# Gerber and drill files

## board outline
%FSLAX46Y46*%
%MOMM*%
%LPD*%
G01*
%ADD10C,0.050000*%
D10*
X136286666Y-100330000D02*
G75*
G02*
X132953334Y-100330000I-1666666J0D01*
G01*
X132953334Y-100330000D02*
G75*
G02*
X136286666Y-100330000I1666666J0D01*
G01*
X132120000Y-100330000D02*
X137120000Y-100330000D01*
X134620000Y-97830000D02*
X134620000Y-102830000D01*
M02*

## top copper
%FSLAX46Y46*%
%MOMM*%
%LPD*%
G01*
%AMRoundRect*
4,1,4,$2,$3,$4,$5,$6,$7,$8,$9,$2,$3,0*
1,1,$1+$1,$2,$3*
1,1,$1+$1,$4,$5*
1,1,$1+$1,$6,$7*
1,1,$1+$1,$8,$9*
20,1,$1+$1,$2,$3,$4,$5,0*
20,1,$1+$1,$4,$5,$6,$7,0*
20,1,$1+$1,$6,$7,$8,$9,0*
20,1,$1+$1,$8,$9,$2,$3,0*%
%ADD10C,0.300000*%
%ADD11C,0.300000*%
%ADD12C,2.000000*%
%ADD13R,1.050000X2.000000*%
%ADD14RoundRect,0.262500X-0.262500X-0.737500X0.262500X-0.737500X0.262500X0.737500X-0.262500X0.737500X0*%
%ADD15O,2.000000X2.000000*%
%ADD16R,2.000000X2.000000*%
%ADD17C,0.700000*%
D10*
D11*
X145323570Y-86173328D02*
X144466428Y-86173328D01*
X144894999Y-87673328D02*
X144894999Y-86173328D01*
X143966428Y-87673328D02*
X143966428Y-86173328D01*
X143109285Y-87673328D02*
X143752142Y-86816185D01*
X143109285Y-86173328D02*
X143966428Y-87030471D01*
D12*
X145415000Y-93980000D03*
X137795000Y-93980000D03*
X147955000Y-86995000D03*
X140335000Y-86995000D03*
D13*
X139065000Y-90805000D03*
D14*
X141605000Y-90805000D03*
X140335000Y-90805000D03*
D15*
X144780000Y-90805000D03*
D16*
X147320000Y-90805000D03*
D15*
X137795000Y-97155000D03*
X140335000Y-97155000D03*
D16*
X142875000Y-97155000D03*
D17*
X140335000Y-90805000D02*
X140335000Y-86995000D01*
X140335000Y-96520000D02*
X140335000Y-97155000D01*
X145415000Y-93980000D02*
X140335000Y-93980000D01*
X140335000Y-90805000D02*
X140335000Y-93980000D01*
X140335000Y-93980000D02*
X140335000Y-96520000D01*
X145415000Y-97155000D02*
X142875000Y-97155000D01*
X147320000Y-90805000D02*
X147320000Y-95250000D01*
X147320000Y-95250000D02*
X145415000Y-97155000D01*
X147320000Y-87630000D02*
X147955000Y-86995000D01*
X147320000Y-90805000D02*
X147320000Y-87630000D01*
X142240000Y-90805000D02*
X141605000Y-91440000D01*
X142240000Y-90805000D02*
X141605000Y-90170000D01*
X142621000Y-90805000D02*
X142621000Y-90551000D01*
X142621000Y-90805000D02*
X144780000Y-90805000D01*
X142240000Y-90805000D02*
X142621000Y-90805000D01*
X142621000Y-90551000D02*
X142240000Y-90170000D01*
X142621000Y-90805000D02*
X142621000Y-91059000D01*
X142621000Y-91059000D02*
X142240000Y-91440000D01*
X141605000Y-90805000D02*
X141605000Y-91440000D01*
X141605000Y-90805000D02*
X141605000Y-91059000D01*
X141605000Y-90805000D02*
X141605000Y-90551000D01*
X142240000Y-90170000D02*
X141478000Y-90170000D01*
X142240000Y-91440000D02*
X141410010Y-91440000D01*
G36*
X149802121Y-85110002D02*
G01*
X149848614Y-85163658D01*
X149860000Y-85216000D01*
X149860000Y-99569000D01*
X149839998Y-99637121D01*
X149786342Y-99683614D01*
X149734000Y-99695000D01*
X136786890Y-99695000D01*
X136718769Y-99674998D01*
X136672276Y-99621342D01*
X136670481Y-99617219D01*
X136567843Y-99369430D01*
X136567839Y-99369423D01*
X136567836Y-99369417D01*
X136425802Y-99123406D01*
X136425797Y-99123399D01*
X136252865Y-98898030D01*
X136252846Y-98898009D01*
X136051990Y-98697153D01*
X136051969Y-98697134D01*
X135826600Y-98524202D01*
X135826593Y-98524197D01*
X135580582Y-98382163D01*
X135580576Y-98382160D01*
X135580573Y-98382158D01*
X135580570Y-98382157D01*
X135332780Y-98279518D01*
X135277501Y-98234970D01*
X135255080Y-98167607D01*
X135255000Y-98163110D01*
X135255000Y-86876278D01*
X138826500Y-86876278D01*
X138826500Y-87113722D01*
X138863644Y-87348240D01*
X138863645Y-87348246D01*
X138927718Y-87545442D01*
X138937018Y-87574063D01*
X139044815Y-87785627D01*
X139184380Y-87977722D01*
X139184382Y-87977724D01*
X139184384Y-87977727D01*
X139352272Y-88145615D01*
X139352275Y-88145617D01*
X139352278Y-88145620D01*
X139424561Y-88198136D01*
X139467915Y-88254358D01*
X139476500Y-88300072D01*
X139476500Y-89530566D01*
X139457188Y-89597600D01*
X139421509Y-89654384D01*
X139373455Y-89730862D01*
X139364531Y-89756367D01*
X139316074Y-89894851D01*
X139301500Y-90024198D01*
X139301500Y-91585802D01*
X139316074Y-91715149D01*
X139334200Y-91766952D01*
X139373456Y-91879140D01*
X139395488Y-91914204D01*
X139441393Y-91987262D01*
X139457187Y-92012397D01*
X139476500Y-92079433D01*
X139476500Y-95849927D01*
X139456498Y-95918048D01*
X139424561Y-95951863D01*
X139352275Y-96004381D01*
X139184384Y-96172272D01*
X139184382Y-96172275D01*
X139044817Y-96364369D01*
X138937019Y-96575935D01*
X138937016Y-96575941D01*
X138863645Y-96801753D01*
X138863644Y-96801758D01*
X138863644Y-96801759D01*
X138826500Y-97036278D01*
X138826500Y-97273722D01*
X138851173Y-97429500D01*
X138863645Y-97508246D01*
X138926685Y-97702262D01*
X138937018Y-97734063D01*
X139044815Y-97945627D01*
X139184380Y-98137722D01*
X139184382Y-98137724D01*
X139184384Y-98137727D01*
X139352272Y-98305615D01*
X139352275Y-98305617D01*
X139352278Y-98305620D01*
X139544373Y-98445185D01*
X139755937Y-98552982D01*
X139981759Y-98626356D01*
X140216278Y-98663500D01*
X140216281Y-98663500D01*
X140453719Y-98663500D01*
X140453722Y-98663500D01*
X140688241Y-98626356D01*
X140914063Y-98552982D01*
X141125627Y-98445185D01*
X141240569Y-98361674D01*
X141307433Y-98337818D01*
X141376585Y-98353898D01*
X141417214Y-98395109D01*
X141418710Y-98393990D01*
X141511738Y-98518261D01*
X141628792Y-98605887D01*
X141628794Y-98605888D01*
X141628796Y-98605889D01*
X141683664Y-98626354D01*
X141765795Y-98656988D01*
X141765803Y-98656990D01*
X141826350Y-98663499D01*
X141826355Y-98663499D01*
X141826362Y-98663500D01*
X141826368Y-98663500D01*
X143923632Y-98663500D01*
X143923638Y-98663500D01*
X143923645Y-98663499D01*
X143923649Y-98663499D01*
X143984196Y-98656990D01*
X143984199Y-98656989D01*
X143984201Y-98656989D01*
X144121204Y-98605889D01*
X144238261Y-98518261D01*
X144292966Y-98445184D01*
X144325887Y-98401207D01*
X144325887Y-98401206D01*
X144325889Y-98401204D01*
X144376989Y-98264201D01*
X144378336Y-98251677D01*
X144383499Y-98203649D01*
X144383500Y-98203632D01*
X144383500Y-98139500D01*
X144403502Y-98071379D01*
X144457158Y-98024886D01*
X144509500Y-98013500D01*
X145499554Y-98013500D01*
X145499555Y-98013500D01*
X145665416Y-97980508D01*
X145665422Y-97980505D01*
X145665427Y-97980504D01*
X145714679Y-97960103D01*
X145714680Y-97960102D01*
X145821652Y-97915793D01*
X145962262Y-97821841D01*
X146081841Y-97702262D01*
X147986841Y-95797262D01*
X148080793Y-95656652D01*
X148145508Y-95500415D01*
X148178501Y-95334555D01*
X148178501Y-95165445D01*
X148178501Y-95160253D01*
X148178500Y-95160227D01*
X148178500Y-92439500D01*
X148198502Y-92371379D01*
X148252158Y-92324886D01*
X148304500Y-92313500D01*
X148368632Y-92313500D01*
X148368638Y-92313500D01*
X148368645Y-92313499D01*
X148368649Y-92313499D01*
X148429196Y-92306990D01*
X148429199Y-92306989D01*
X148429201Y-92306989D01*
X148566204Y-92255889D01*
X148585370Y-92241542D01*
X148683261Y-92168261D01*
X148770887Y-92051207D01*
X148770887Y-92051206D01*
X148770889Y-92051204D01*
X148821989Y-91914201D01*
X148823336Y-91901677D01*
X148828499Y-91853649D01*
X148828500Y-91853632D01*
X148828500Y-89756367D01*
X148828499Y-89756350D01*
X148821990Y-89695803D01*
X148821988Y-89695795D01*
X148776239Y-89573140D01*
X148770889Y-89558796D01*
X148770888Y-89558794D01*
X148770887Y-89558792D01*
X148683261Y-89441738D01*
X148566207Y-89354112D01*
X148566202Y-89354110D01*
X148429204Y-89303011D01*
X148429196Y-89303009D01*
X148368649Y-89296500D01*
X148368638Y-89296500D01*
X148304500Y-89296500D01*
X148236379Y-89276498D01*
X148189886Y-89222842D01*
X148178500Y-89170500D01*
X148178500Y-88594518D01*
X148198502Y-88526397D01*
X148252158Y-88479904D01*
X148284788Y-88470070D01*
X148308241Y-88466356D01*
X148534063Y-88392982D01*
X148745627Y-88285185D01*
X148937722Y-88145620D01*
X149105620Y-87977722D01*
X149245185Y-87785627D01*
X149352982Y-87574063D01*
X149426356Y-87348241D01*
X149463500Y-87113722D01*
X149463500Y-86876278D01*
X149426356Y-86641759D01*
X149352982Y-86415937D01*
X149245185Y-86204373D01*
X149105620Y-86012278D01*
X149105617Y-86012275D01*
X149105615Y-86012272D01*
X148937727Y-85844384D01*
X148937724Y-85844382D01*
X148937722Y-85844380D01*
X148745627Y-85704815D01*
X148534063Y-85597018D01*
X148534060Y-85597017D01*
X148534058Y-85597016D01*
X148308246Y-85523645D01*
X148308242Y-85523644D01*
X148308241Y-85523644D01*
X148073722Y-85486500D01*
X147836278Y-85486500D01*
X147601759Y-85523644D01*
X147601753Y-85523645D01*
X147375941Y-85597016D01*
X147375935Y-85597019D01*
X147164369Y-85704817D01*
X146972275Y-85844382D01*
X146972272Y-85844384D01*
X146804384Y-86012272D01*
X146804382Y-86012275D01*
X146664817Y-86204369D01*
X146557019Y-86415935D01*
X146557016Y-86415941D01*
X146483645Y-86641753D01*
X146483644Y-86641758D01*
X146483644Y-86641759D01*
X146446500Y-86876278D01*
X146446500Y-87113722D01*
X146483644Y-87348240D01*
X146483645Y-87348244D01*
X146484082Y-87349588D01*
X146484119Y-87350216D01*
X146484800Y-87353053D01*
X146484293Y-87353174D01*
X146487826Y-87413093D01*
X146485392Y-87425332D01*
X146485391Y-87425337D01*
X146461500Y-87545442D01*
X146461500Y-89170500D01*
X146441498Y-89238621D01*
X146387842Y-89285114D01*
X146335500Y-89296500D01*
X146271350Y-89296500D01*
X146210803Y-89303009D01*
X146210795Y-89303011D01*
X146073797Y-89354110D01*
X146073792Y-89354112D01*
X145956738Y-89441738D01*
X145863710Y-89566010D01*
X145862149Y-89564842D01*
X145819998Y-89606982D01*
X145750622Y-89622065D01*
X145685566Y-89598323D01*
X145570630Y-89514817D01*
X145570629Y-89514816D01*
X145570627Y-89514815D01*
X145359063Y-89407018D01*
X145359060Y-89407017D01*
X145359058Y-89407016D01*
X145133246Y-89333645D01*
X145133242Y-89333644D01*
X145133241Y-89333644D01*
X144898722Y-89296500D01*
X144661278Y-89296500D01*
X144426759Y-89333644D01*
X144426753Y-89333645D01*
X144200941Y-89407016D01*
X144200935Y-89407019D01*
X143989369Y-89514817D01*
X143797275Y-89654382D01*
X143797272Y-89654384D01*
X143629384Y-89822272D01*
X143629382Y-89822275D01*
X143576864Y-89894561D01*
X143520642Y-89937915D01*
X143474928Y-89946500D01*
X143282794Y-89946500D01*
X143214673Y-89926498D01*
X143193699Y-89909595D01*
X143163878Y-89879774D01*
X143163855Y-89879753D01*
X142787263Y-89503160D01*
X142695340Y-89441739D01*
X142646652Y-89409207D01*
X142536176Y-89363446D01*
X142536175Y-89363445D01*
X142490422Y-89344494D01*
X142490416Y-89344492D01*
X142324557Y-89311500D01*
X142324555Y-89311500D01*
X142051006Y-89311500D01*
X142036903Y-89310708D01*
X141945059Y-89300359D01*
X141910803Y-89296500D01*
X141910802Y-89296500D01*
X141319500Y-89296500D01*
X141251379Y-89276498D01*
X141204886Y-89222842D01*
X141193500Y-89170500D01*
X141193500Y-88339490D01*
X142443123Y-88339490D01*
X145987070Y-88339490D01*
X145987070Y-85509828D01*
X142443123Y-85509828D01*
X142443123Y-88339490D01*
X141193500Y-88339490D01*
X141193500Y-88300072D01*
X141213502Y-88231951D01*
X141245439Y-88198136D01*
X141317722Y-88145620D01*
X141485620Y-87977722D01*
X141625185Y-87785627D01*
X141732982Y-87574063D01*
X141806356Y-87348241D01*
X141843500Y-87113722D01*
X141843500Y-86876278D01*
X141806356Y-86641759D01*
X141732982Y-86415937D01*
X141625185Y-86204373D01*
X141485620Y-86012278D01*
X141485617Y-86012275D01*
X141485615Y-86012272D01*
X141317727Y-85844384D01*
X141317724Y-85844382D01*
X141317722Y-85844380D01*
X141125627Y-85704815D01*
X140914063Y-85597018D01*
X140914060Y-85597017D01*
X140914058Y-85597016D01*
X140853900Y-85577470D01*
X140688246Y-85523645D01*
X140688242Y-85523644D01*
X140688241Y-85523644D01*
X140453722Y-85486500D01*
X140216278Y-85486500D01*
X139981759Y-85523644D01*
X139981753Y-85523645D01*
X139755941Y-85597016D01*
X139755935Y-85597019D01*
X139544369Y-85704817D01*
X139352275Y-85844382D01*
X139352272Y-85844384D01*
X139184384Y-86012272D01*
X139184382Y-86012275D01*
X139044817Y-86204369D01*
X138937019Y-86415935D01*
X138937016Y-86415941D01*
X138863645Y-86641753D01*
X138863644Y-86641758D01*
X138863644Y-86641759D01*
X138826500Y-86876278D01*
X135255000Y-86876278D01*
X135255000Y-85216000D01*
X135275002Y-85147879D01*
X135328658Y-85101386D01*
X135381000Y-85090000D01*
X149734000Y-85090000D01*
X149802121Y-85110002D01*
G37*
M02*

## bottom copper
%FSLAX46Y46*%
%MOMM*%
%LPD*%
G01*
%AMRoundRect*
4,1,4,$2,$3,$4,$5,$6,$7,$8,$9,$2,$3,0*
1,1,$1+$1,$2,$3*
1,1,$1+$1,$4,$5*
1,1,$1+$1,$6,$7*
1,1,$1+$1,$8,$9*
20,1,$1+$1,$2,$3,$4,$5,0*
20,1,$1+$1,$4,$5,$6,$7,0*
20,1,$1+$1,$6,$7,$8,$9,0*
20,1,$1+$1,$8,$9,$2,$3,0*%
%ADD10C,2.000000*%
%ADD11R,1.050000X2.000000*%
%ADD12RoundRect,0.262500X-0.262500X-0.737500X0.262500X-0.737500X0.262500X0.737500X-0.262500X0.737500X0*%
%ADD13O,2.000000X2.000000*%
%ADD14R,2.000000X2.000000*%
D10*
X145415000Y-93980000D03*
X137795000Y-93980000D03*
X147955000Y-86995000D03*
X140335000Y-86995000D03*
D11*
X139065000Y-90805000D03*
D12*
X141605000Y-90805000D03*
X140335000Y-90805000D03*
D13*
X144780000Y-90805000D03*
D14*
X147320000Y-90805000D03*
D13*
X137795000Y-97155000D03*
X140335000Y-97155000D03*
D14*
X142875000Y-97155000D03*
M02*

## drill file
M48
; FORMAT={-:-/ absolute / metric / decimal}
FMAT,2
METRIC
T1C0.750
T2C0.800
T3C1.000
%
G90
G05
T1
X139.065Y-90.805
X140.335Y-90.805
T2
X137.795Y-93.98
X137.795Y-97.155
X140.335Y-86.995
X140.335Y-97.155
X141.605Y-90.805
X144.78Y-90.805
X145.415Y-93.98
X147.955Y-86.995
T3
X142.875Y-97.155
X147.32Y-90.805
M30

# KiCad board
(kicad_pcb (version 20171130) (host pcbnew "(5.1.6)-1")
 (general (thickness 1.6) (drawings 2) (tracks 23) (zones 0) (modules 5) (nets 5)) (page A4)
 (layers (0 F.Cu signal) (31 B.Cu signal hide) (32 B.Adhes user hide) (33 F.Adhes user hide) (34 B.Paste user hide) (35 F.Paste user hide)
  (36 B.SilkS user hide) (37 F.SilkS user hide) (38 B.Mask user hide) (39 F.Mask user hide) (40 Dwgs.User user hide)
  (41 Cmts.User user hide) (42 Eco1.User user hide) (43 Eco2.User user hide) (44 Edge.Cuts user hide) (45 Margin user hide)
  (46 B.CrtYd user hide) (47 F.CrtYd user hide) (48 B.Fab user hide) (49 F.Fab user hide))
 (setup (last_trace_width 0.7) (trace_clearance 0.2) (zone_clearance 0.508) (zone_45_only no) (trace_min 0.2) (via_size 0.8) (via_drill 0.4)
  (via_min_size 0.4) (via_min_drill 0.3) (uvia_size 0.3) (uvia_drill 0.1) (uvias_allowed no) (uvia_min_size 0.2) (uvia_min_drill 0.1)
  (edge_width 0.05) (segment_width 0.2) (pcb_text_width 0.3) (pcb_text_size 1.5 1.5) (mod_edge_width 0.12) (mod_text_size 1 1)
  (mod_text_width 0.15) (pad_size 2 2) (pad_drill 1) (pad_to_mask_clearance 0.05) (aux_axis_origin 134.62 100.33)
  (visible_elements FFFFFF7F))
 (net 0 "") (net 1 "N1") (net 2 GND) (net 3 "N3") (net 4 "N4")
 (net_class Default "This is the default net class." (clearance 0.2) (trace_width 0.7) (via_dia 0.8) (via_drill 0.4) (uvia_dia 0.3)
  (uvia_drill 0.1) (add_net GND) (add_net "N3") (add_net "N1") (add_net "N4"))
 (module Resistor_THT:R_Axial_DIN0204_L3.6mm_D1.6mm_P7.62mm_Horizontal (layer F.Cu) (at 137.795 93.98)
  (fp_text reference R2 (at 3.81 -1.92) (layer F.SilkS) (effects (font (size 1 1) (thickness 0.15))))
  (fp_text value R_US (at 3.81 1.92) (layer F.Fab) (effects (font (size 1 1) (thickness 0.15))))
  (pad 2 thru_hole circle (at 7.62 0) (size 2 2) (drill 0.8) (layers *.Cu *.Mask) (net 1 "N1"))
  (pad 1 thru_hole circle (at 0 0) (size 2 2) (drill 0.8) (layers *.Cu *.Mask) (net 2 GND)))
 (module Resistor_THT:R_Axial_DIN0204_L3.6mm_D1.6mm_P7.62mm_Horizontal (layer F.Cu) (at 140.335 86.995)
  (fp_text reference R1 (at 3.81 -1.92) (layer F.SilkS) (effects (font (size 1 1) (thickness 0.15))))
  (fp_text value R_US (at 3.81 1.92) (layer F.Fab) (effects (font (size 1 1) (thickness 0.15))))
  (pad 2 thru_hole circle (at 7.62 0) (size 2 2) (drill 0.8) (layers *.Cu *.Mask) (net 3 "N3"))
  (pad 1 thru_hole circle (at 0 0) (size 2 2) (drill 0.8) (layers *.Cu *.Mask) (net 1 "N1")))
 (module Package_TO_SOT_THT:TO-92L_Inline (layer F.Cu) (at 139.065 90.805)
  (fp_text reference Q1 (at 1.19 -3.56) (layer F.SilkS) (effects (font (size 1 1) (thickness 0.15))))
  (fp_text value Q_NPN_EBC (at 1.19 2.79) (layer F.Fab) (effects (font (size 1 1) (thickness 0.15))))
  (pad 1 thru_hole rect (at 0 0) (size 1.05 2) (drill 0.75) (layers *.Cu *.Mask) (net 2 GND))
  (pad 3 thru_hole roundrect (at 2.54 0) (size 1.05 2) (drill 0.8) (layers *.Cu *.Mask) (roundrect_rratio 0.25) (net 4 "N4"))
  (pad 2 thru_hole roundrect (at 1.27 0) (size 1.05 2) (drill 0.75) (layers *.Cu *.Mask) (roundrect_rratio 0.25) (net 1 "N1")))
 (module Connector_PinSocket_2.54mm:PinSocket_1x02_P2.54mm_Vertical (layer F.Cu) (at 147.32 90.805 270)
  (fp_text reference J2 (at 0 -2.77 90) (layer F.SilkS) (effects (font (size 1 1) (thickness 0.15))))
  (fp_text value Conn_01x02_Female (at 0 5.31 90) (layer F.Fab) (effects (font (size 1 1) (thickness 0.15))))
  (pad 2 thru_hole oval (at 0 2.54 270) (size 2 2) (drill 0.8) (layers *.Cu *.Mask) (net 4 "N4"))
  (pad 1 thru_hole rect (at 0 0 270) (size 2 2) (drill 1) (layers *.Cu *.Mask) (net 3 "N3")))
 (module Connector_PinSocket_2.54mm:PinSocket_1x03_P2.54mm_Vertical (layer F.Cu) (at 142.875 97.155 270)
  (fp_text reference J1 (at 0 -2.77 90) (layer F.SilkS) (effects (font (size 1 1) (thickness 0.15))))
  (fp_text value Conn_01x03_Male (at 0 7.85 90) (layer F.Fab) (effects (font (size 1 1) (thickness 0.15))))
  (pad 3 thru_hole oval (at 0 5.08 270) (size 2 2) (drill 0.8) (layers *.Cu *.Mask) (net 2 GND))
  (pad 2 thru_hole oval (at 0 2.54 270) (size 2 2) (drill 0.8) (layers *.Cu *.Mask) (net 1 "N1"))
  (pad 1 thru_hole rect (at 0 0 270) (size 2 2) (drill 1) (layers *.Cu *.Mask) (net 3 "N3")))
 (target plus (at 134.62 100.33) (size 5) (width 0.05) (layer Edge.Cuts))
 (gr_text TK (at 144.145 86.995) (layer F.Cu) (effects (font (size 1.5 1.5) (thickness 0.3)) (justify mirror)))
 (segment (start 140.335 90.805) (end 140.335 86.995) (width 0.7) (layer F.Cu) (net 1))
 (segment (start 140.335 96.52) (end 140.335 97.155) (width 0.7) (layer F.Cu) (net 1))
 (segment (start 145.415 93.98) (end 140.335 93.98) (width 0.7) (layer F.Cu) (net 1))
 (segment (start 140.335 90.805) (end 140.335 93.98) (width 0.7) (layer F.Cu) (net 1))
 (segment (start 140.335 93.98) (end 140.335 96.52) (width 0.7) (layer F.Cu) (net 1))
 (segment (start 145.415 97.155) (end 142.875 97.155) (width 0.7) (layer F.Cu) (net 3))
 (segment (start 147.32 90.805) (end 147.32 95.25) (width 0.7) (layer F.Cu) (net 3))
 (segment (start 147.32 95.25) (end 145.415 97.155) (width 0.7) (layer F.Cu) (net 3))
 (segment (start 147.32 87.63) (end 147.955 86.995) (width 0.7) (layer F.Cu) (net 3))
 (segment (start 147.32 90.805) (end 147.32 87.63) (width 0.7) (layer F.Cu) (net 3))
 (segment (start 142.24 90.805) (end 141.605 91.44) (width 0.7) (layer F.Cu) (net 4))
 (segment (start 142.24 90.805) (end 141.605 90.17) (width 0.7) (layer F.Cu) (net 4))
 (segment (start 142.621 90.805) (end 142.621 90.551) (width 0.7) (layer F.Cu) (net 4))
 (segment (start 142.621 90.805) (end 144.78 90.805) (width 0.7) (layer F.Cu) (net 4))
 (segment (start 142.24 90.805) (end 142.621 90.805) (width 0.7) (layer F.Cu) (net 4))
 (segment (start 142.621 90.551) (end 142.24 90.17) (width 0.7) (layer F.Cu) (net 4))
 (segment (start 142.621 90.805) (end 142.621 91.059) (width 0.7) (layer F.Cu) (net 4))
 (segment (start 142.621 91.059) (end 142.24 91.44) (width 0.7) (layer F.Cu) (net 4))
 (segment (start 141.605 90.805) (end 141.605 91.44) (width 0.7) (layer F.Cu) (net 4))
 (segment (start 141.605 90.805) (end 141.605 91.059) (width 0.7) (layer F.Cu) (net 4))
 (segment (start 141.605 90.805) (end 141.605 90.551) (width 0.7) (layer F.Cu) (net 4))
 (segment (start 142.24 90.17) (end 141.478 90.17) (width 0.7) (layer F.Cu) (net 4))
 (segment (start 142.24 91.44) (end 141.41001 91.44) (width 0.7) (layer F.Cu) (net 4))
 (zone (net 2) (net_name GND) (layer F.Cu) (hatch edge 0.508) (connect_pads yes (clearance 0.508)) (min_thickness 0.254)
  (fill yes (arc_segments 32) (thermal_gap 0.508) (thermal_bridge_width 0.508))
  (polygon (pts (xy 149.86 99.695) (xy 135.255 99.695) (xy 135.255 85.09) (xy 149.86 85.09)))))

